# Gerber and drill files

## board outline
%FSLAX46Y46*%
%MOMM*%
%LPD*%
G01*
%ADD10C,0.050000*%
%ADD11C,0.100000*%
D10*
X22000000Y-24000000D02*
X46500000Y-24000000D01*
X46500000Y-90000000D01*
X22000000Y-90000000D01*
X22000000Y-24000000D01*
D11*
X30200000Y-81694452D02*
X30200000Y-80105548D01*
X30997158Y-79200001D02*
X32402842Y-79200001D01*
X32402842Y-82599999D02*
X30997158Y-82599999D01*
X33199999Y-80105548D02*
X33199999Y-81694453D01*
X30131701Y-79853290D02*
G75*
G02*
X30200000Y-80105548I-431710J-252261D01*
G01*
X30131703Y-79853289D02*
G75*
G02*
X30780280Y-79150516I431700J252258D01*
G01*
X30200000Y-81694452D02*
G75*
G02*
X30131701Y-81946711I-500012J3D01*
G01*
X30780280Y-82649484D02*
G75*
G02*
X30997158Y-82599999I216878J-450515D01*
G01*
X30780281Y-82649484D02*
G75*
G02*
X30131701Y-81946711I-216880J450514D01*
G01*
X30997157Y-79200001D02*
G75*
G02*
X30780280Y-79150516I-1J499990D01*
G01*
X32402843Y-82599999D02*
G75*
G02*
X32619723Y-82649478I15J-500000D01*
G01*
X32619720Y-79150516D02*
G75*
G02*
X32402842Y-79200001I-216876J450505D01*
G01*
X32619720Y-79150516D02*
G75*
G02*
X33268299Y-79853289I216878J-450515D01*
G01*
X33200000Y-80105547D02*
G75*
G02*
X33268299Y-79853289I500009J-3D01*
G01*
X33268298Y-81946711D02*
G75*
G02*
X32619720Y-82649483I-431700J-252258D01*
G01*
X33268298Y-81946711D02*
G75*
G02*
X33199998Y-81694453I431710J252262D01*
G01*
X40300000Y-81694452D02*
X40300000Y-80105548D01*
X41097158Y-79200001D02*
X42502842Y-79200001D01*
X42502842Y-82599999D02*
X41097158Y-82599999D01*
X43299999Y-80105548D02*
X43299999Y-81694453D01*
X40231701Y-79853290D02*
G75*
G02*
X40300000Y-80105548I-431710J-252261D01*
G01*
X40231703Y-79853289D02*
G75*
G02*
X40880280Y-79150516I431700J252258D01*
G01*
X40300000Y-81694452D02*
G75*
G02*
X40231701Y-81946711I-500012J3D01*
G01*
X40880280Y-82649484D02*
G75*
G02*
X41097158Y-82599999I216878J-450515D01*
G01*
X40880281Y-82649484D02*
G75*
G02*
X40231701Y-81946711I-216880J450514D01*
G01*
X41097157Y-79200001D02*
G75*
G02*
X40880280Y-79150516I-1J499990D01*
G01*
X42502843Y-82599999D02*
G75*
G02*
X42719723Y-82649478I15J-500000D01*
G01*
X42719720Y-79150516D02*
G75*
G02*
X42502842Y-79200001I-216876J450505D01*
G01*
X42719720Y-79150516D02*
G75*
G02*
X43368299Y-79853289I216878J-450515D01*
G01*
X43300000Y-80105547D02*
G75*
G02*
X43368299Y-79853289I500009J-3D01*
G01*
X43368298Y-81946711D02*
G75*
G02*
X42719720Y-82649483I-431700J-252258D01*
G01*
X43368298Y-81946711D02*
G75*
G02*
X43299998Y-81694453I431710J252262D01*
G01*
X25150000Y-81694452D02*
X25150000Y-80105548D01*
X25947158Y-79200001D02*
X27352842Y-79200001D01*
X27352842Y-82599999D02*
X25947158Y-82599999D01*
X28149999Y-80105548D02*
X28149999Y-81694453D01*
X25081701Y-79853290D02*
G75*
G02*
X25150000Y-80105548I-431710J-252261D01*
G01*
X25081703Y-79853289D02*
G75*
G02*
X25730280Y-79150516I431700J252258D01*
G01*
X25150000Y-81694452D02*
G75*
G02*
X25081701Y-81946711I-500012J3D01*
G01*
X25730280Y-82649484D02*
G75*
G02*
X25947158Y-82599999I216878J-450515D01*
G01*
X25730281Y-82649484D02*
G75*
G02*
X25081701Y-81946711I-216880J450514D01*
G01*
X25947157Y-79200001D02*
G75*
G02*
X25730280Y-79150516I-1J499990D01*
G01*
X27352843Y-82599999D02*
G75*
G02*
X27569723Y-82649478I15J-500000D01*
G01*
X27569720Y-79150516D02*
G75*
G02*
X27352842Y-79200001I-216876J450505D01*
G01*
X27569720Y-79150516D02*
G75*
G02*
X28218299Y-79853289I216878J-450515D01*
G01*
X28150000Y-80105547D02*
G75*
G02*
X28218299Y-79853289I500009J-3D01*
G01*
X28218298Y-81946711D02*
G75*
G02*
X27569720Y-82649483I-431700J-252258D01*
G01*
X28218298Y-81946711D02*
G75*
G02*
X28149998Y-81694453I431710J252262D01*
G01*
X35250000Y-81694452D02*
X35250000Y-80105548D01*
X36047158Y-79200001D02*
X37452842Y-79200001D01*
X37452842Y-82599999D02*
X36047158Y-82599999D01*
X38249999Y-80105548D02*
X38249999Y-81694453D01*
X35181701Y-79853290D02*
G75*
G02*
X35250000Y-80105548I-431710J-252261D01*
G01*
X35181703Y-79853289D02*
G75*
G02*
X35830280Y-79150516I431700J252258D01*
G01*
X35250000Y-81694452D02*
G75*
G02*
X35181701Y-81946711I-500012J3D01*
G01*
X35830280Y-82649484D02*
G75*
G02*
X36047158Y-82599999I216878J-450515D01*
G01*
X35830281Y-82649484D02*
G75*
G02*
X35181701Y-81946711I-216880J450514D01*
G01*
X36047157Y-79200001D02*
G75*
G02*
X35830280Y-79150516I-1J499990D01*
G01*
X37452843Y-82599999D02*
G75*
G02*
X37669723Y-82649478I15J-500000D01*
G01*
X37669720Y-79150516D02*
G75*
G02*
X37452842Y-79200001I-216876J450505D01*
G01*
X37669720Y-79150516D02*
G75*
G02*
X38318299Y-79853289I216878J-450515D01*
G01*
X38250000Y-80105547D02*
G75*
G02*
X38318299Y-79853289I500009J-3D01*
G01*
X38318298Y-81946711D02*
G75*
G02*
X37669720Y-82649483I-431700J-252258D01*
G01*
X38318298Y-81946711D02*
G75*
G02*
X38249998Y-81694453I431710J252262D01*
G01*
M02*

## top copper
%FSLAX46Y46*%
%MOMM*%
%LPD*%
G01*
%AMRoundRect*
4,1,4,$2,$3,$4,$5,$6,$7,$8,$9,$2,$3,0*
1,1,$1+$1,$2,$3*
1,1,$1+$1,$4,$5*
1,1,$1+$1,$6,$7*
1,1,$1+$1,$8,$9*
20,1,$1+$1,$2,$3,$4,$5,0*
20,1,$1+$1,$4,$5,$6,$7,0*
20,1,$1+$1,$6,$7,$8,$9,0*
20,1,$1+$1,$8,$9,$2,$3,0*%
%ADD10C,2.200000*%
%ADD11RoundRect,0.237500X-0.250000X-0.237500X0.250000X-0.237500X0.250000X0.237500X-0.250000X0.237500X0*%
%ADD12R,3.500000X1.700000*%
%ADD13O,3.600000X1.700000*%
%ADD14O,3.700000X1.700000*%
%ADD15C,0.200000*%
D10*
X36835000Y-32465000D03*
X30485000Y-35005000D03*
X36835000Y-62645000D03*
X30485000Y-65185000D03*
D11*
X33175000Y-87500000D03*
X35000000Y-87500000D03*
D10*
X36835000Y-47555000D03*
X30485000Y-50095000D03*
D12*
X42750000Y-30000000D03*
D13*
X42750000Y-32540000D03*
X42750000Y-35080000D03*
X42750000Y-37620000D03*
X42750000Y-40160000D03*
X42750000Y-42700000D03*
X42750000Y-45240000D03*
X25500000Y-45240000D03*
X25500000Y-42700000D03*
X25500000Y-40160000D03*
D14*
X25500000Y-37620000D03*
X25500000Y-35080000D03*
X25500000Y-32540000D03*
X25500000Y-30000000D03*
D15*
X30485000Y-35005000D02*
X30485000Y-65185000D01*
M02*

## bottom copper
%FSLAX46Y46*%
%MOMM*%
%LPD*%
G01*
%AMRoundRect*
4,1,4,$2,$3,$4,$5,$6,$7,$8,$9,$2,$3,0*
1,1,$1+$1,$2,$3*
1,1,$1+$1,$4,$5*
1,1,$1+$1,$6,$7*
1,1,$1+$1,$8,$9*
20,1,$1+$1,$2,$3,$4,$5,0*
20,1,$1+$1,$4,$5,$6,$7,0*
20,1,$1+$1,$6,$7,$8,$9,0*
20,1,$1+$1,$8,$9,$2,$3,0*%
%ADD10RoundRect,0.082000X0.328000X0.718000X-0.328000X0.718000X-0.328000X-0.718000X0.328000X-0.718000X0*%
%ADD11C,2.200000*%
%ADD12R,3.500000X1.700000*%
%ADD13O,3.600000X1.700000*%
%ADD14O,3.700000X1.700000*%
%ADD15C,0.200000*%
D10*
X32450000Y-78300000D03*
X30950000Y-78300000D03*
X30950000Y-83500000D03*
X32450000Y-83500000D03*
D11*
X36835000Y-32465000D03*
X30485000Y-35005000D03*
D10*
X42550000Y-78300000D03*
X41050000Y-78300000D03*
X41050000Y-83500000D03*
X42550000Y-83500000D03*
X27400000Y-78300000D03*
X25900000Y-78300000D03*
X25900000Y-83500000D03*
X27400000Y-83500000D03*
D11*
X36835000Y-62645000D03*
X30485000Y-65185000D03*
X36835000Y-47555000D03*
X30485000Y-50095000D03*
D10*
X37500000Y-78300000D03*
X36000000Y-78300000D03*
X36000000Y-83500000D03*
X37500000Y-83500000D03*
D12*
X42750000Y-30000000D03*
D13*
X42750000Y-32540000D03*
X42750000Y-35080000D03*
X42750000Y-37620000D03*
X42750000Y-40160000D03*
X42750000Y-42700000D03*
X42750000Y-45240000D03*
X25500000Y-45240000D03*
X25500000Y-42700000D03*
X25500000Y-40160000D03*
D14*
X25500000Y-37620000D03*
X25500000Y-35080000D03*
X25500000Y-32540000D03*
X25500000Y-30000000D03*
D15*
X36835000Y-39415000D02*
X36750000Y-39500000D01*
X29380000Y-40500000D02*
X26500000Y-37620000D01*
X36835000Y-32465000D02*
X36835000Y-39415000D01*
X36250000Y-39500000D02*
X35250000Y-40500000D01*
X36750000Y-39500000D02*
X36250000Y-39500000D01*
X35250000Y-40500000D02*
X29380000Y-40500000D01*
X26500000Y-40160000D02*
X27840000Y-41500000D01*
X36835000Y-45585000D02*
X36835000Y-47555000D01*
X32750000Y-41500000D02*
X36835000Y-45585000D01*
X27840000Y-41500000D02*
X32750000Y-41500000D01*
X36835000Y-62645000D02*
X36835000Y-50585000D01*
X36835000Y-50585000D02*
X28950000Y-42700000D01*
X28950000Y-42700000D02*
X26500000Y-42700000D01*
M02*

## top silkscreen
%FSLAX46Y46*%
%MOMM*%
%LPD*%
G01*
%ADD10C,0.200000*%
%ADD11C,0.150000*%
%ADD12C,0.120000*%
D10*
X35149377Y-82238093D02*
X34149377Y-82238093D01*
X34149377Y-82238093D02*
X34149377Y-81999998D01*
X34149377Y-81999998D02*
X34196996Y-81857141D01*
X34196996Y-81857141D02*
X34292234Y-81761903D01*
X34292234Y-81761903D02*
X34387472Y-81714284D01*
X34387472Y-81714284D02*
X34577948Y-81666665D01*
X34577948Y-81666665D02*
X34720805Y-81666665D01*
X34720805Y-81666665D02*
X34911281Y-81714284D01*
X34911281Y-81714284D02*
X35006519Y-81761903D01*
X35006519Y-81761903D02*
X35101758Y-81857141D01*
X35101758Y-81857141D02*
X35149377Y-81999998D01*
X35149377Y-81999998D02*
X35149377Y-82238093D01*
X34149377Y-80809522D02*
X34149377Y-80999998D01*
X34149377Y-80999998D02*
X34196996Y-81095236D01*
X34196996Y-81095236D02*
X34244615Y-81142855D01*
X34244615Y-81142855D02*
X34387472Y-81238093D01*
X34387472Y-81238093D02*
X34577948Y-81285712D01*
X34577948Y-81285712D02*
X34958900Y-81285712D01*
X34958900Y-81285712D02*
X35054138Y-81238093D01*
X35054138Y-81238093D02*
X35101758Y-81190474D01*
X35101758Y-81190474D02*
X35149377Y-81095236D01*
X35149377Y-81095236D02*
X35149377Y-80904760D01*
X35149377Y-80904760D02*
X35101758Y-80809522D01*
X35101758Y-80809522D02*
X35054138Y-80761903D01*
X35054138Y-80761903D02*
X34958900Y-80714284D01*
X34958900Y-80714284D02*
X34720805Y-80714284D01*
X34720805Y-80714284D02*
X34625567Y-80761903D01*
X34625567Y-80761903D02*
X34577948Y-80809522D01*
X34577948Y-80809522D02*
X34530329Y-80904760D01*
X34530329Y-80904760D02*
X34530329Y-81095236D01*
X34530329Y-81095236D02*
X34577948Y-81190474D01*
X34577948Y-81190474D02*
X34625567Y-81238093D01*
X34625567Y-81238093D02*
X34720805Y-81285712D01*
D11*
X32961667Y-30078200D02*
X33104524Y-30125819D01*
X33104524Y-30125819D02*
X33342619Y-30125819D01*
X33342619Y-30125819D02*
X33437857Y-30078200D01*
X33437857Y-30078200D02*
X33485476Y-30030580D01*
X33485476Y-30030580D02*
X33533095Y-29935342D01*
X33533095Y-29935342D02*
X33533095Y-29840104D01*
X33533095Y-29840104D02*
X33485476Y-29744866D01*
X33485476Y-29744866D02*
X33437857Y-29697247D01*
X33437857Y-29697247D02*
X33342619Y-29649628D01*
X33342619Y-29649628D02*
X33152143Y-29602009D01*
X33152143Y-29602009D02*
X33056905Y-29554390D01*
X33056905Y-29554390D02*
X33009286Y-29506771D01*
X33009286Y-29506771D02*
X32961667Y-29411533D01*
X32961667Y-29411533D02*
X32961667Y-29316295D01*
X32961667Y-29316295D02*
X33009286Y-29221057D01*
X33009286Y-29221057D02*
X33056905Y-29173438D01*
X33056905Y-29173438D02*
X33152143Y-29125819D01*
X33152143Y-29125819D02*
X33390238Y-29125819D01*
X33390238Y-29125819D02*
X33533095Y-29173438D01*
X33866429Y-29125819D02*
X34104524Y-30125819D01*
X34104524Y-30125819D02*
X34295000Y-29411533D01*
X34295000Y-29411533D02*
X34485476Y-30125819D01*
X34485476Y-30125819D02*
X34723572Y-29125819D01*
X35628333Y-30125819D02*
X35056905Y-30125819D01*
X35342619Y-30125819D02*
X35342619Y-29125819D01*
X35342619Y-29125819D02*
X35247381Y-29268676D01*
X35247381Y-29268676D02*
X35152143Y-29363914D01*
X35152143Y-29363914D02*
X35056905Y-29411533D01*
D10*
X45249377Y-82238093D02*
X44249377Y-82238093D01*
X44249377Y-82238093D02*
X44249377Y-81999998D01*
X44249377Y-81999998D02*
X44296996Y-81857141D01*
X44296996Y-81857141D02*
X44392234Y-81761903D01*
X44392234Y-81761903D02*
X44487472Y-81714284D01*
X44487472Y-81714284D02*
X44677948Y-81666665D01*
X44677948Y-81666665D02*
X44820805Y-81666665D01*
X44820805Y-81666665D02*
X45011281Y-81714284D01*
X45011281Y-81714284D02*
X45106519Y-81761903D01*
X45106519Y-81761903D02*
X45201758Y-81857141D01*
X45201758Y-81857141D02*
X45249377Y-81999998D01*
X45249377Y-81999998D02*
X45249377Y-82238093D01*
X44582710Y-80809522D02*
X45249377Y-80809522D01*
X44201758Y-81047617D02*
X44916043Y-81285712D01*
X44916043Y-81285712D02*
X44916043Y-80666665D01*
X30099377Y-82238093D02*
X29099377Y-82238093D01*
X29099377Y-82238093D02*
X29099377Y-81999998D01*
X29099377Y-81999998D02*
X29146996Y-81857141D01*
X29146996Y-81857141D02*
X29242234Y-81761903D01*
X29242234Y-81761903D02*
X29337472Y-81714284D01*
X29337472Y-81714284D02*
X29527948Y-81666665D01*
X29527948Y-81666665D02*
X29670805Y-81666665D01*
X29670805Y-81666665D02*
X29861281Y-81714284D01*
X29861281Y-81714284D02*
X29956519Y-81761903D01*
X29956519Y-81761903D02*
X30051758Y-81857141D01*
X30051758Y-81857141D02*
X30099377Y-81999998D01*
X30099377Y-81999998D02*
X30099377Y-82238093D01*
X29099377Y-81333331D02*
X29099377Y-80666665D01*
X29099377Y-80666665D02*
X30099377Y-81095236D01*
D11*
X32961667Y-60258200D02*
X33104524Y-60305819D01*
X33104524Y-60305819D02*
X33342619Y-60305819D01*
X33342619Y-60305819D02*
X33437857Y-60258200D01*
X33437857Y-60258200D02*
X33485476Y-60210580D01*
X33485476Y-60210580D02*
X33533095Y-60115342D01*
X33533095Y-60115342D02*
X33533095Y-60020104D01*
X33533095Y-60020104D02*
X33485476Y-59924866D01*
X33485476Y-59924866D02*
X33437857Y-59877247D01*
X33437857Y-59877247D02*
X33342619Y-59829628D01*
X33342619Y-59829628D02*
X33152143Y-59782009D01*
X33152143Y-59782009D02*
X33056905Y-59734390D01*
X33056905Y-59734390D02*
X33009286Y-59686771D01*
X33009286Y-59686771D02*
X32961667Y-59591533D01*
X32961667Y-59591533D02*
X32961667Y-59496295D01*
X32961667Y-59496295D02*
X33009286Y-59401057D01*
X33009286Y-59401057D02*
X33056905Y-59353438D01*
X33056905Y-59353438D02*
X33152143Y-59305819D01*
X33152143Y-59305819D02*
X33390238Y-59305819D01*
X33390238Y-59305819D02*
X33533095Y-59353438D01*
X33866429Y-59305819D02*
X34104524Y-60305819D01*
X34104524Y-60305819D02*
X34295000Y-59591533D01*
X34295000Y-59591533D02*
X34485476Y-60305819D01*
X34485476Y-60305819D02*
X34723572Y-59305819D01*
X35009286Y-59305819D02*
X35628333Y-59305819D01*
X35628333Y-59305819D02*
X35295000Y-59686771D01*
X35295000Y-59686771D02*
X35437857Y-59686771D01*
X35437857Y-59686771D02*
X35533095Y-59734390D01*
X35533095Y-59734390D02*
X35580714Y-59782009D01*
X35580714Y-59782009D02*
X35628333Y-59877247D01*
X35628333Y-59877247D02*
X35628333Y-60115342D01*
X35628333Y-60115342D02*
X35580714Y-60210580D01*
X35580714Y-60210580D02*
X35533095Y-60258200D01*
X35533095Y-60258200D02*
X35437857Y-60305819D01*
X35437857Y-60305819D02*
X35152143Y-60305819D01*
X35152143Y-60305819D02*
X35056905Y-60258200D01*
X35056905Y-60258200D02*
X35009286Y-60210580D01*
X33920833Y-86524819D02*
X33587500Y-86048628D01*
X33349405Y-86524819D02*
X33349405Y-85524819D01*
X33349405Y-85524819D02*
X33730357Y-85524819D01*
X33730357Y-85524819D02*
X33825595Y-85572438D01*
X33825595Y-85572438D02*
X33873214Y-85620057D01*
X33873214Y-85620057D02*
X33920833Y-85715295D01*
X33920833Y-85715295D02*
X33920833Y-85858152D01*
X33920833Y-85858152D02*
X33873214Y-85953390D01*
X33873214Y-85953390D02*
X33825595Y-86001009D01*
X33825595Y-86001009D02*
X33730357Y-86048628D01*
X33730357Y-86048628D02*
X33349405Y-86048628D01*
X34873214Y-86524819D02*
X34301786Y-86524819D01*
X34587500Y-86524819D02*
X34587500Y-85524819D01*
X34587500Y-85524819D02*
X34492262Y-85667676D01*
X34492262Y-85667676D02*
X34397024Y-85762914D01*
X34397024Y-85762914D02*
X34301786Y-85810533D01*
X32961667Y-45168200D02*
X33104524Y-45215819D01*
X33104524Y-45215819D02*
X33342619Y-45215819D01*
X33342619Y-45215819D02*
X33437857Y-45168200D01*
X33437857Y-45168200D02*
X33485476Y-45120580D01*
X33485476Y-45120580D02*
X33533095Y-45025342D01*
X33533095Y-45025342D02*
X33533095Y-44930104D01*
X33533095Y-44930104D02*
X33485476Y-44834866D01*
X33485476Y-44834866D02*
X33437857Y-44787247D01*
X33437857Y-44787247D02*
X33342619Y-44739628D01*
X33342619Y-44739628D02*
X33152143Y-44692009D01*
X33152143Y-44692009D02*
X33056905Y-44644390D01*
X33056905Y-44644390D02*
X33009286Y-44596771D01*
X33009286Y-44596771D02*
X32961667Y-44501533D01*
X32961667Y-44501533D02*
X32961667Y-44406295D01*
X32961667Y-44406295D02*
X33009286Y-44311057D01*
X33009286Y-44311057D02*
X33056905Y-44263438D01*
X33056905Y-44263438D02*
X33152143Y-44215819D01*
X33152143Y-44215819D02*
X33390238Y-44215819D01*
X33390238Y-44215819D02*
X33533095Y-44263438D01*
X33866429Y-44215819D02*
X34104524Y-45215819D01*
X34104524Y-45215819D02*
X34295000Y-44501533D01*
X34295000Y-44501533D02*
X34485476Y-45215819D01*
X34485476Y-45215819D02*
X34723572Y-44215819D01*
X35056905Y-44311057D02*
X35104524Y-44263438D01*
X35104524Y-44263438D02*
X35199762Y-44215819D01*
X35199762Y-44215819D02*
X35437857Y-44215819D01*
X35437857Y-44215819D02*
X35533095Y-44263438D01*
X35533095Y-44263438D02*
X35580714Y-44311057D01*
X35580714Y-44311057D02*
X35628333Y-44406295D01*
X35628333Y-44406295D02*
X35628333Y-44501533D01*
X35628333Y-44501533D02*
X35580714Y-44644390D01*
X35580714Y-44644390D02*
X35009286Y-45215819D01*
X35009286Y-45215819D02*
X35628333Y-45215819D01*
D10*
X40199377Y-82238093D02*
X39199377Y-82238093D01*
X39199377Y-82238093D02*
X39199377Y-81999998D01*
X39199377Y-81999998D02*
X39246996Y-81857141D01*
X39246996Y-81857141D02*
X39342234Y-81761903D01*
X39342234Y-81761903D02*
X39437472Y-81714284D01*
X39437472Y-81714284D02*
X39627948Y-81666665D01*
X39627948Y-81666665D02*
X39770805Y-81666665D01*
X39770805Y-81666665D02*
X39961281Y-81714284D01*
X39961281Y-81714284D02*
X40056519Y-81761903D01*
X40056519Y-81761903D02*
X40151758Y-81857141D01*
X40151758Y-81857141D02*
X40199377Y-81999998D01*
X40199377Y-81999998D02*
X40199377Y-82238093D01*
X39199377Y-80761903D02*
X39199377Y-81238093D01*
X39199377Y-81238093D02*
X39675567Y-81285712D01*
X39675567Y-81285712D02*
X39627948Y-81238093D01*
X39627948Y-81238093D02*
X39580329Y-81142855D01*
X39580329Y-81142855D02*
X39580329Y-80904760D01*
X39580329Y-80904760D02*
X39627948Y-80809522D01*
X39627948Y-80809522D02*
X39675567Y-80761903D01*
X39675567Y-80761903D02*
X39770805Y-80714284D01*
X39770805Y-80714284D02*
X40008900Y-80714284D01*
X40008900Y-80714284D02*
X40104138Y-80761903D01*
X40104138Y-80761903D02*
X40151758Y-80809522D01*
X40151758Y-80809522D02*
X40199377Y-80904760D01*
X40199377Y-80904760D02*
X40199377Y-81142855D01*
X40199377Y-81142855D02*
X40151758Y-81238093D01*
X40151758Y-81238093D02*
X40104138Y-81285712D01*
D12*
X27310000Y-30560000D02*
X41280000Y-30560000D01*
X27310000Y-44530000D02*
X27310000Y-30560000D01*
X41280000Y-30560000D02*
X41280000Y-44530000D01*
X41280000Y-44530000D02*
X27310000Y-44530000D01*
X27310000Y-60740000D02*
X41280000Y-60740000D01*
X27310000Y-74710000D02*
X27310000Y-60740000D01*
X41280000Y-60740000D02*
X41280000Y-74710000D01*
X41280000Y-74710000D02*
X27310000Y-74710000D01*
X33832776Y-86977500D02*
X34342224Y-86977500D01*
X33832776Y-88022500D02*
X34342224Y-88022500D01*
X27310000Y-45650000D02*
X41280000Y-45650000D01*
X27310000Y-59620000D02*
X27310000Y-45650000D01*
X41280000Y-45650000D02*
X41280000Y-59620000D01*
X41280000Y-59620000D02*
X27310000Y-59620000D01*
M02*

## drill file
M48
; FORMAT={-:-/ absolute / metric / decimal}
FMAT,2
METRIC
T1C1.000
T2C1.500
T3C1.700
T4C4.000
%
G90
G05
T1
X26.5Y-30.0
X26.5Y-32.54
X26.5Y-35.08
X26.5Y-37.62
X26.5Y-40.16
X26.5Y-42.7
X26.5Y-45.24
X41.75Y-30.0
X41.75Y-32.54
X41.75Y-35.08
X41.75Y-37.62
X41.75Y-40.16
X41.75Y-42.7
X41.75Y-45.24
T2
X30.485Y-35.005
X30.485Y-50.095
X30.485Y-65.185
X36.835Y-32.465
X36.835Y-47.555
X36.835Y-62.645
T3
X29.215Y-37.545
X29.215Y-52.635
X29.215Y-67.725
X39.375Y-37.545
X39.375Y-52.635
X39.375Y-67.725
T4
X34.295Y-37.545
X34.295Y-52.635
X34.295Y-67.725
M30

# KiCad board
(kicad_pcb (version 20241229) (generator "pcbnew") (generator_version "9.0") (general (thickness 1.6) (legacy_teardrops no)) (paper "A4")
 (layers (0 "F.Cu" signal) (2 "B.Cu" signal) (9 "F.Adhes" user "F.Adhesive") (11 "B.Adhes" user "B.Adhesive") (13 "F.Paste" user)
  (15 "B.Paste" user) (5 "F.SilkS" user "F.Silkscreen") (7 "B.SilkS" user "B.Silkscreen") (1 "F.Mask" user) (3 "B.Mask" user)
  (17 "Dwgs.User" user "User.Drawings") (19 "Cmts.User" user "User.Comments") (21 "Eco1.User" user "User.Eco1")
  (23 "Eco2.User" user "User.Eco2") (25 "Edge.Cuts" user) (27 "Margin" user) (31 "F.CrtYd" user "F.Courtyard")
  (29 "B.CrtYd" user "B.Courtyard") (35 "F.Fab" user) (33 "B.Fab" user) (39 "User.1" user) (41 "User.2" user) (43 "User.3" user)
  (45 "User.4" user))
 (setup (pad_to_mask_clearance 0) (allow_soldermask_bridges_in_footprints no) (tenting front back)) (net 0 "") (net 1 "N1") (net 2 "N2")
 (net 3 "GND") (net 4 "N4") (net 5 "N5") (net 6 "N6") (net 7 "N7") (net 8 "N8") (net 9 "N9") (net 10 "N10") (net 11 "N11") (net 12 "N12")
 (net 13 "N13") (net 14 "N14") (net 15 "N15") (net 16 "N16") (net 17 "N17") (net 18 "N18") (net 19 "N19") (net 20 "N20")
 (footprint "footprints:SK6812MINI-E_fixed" (layer "F.Cu") (at 31.597158 80.899999 -90)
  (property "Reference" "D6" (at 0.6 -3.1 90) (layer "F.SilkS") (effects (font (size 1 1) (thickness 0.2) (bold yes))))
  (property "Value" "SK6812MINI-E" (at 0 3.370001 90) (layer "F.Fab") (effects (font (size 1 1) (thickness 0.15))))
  (fp_line (start 0.794453 1.397158) (end -0.794451 1.397158) (stroke (width 0.1) (type solid)) (layer "Edge.Cuts"))
  (fp_line (start -1.699998 0.6) (end -1.699998 -0.805684) (stroke (width 0.1) (type solid)) (layer "Edge.Cuts"))
  (fp_line (start 1.7 -0.805684) (end 1.7 0.6) (stroke (width 0.1) (type solid)) (layer "Edge.Cuts"))
  (fp_line (start -0.794451 -1.602841) (end 0.794454 -1.602841) (stroke (width 0.1) (type solid)) (layer "Edge.Cuts"))
  (fp_arc (start -1.046709 1.465457) (mid -0.925121 1.414535) (end -0.794451 1.397158) (stroke (width 0.1) (type solid)) (layer "Edge.Cuts"))
  (fp_arc (start -1.04671 1.465455) (mid -1.638069 1.401192) (end -1.749483 0.816878) (stroke (width 0.1) (type solid)) (layer "Edge.Cuts"))
  (fp_arc (start 0.794453 1.397158) (mid 0.925124 1.414535) (end 1.046712 1.465457) (stroke (width 0.1) (type solid)) (layer "Edge.Cuts"))
  (fp_arc (start 1.749485 0.816878) (mid 1.712528 0.711226) (end 1.7 0.6) (stroke (width 0.1) (type solid)) (layer "Edge.Cuts"))
  (fp_arc (start 1.749485 0.816877) (mid 1.638073 1.401193) (end 1.046712 1.465457) (stroke (width 0.1) (type solid)) (layer "Edge.Cuts"))
  (fp_arc (start -1.699998 0.600001) (mid -1.712526 0.711226) (end -1.749483 0.816878) (stroke (width 0.1) (type solid)) (layer "Edge.Cuts"))
  (fp_arc (start 1.7 -0.805685) (mid 1.712528 -0.91691) (end 1.749485 -1.022562) (stroke (width 0.1) (type solid)) (layer "Edge.Cuts"))
  (fp_arc (start -1.749483 -1.022562) (mid -1.712526 -0.91691) (end -1.699998 -0.805684) (stroke (width 0.1) (type solid))
   (layer "Edge.Cuts"))
  (fp_arc (start -1.749483 -1.022562) (mid -1.63807 -1.606877) (end -1.04671 -1.671141) (stroke (width 0.1) (type solid))
   (layer "Edge.Cuts"))
  (fp_arc (start -0.794452 -1.602842) (mid -0.925122 -1.620219) (end -1.04671 -1.671141) (stroke (width 0.1) (type solid))
   (layer "Edge.Cuts"))
  (fp_arc (start 1.046712 -1.67114) (mid 1.638072 -1.606876) (end 1.749485 -1.022562) (stroke (width 0.1) (type solid)) (layer "Edge.Cuts"))
  (fp_arc (start 1.046712 -1.67114) (mid 0.925124 -1.620218) (end 0.794454 -1.602841) (stroke (width 0.1) (type solid)) (layer "Edge.Cuts"))
  (pad "1" smd roundrect (at -2.599999 -0.852842 180) (size 0.82 1.6) (layers "B.Cu" "B.Mask" "B.Paste") (roundrect_rratio 0.1) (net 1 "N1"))
  (pad "2" smd roundrect (at -2.599999 0.647158 180) (size 0.82 1.6) (layers "B.Cu" "B.Mask" "B.Paste") (roundrect_rratio 0.1) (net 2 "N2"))
  (pad "3" smd roundrect (at 2.600001 0.647158 180) (size 0.82 1.6) (layers "B.Cu" "B.Mask" "B.Paste") (roundrect_rratio 0.1) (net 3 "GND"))
  (pad "4" smd roundrect (at 2.600001 -0.852842 180) (size 0.82 1.6) (layers "B.Cu" "B.Mask" "B.Paste") (roundrect_rratio 0.1) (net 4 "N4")))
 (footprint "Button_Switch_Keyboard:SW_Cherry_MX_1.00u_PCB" (layer "F.Cu") (at 36.835 32.465)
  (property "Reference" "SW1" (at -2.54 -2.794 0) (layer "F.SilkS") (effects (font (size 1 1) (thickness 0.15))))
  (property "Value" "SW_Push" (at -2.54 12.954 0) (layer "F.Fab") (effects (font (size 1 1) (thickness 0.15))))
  (fp_line (start -9.525 -1.905) (end 4.445 -1.905) (stroke (width 0.12) (type solid)) (layer "F.SilkS"))
  (fp_line (start -9.525 12.065) (end -9.525 -1.905) (stroke (width 0.12) (type solid)) (layer "F.SilkS"))
  (fp_line (start 4.445 -1.905) (end 4.445 12.065) (stroke (width 0.12) (type solid)) (layer "F.SilkS"))
  (fp_line (start 4.445 12.065) (end -9.525 12.065) (stroke (width 0.12) (type solid)) (layer "F.SilkS"))
  (pad "" np_thru_hole circle (at -7.62 5.08) (size 1.7 1.7) (drill 1.7) (layers "*.Cu" "*.Mask"))
  (pad "" np_thru_hole circle (at -2.54 5.08) (size 4 4) (drill 4) (layers "*.Cu" "*.Mask"))
  (pad "" np_thru_hole circle (at 2.54 5.08) (size 1.7 1.7) (drill 1.7) (layers "*.Cu" "*.Mask"))
  (pad "1" thru_hole circle (at 0 0) (size 2.2 2.2) (drill 1.5) (layers "*.Cu" "*.Mask") (remove_unused_layers no) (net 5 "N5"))
  (pad "2" thru_hole circle (at -6.35 2.54) (size 2.2 2.2) (drill 1.5) (layers "*.Cu" "*.Mask") (remove_unused_layers no) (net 3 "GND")))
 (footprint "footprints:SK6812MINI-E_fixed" (layer "F.Cu") (at 41.697158 80.899999 -90)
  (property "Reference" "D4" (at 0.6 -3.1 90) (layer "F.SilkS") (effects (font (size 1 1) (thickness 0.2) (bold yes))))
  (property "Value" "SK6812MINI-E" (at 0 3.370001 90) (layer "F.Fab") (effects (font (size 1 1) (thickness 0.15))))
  (fp_line (start 0.794453 1.397158) (end -0.794451 1.397158) (stroke (width 0.1) (type solid)) (layer "Edge.Cuts"))
  (fp_line (start -1.699998 0.6) (end -1.699998 -0.805684) (stroke (width 0.1) (type solid)) (layer "Edge.Cuts"))
  (fp_line (start 1.7 -0.805684) (end 1.7 0.6) (stroke (width 0.1) (type solid)) (layer "Edge.Cuts"))
  (fp_line (start -0.794451 -1.602841) (end 0.794454 -1.602841) (stroke (width 0.1) (type solid)) (layer "Edge.Cuts"))
  (fp_arc (start -1.046709 1.465457) (mid -0.925121 1.414535) (end -0.794451 1.397158) (stroke (width 0.1) (type solid)) (layer "Edge.Cuts"))
  (fp_arc (start -1.04671 1.465455) (mid -1.638069 1.401192) (end -1.749483 0.816878) (stroke (width 0.1) (type solid)) (layer "Edge.Cuts"))
  (fp_arc (start 0.794453 1.397158) (mid 0.925124 1.414535) (end 1.046712 1.465457) (stroke (width 0.1) (type solid)) (layer "Edge.Cuts"))
  (fp_arc (start 1.749485 0.816878) (mid 1.712528 0.711226) (end 1.7 0.6) (stroke (width 0.1) (type solid)) (layer "Edge.Cuts"))
  (fp_arc (start 1.749485 0.816877) (mid 1.638073 1.401193) (end 1.046712 1.465457) (stroke (width 0.1) (type solid)) (layer "Edge.Cuts"))
  (fp_arc (start -1.699998 0.600001) (mid -1.712526 0.711226) (end -1.749483 0.816878) (stroke (width 0.1) (type solid)) (layer "Edge.Cuts"))
  (fp_arc (start 1.7 -0.805685) (mid 1.712528 -0.91691) (end 1.749485 -1.022562) (stroke (width 0.1) (type solid)) (layer "Edge.Cuts"))
  (fp_arc (start -1.749483 -1.022562) (mid -1.712526 -0.91691) (end -1.699998 -0.805684) (stroke (width 0.1) (type solid))
   (layer "Edge.Cuts"))
  (fp_arc (start -1.749483 -1.022562) (mid -1.63807 -1.606877) (end -1.04671 -1.671141) (stroke (width 0.1) (type solid))
   (layer "Edge.Cuts"))
  (fp_arc (start -0.794452 -1.602842) (mid -0.925122 -1.620219) (end -1.04671 -1.671141) (stroke (width 0.1) (type solid))
   (layer "Edge.Cuts"))
  (fp_arc (start 1.046712 -1.67114) (mid 1.638072 -1.606876) (end 1.749485 -1.022562) (stroke (width 0.1) (type solid)) (layer "Edge.Cuts"))
  (fp_arc (start 1.046712 -1.67114) (mid 0.925124 -1.620218) (end 0.794454 -1.602841) (stroke (width 0.1) (type solid)) (layer "Edge.Cuts"))
  (pad "1" smd roundrect (at -2.599999 -0.852842 180) (size 0.82 1.6) (layers "B.Cu" "B.Mask" "B.Paste") (roundrect_rratio 0.1) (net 1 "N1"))
  (pad "2" smd roundrect (at -2.599999 0.647158 180) (size 0.82 1.6) (layers "B.Cu" "B.Mask" "B.Paste") (roundrect_rratio 0.1) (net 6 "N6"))
  (pad "3" smd roundrect (at 2.600001 0.647158 180) (size 0.82 1.6) (layers "B.Cu" "B.Mask" "B.Paste") (roundrect_rratio 0.1) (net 3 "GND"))
  (pad "4" smd roundrect (at 2.600001 -0.852842 180) (size 0.82 1.6) (layers "B.Cu" "B.Mask" "B.Paste") (roundrect_rratio 0.1) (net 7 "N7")))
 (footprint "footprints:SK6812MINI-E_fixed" (layer "F.Cu") (at 26.547158 80.899999 -90)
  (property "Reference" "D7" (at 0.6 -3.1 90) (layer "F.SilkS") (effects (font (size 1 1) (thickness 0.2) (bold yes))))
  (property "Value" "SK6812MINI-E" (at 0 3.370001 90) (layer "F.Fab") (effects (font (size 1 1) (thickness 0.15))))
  (fp_line (start 0.794453 1.397158) (end -0.794451 1.397158) (stroke (width 0.1) (type solid)) (layer "Edge.Cuts"))
  (fp_line (start -1.699998 0.6) (end -1.699998 -0.805684) (stroke (width 0.1) (type solid)) (layer "Edge.Cuts"))
  (fp_line (start 1.7 -0.805684) (end 1.7 0.6) (stroke (width 0.1) (type solid)) (layer "Edge.Cuts"))
  (fp_line (start -0.794451 -1.602841) (end 0.794454 -1.602841) (stroke (width 0.1) (type solid)) (layer "Edge.Cuts"))
  (fp_arc (start -1.046709 1.465457) (mid -0.925121 1.414535) (end -0.794451 1.397158) (stroke (width 0.1) (type solid)) (layer "Edge.Cuts"))
  (fp_arc (start -1.04671 1.465455) (mid -1.638069 1.401192) (end -1.749483 0.816878) (stroke (width 0.1) (type solid)) (layer "Edge.Cuts"))
  (fp_arc (start 0.794453 1.397158) (mid 0.925124 1.414535) (end 1.046712 1.465457) (stroke (width 0.1) (type solid)) (layer "Edge.Cuts"))
  (fp_arc (start 1.749485 0.816878) (mid 1.712528 0.711226) (end 1.7 0.6) (stroke (width 0.1) (type solid)) (layer "Edge.Cuts"))
  (fp_arc (start 1.749485 0.816877) (mid 1.638073 1.401193) (end 1.046712 1.465457) (stroke (width 0.1) (type solid)) (layer "Edge.Cuts"))
  (fp_arc (start -1.699998 0.600001) (mid -1.712526 0.711226) (end -1.749483 0.816878) (stroke (width 0.1) (type solid)) (layer "Edge.Cuts"))
  (fp_arc (start 1.7 -0.805685) (mid 1.712528 -0.91691) (end 1.749485 -1.022562) (stroke (width 0.1) (type solid)) (layer "Edge.Cuts"))
  (fp_arc (start -1.749483 -1.022562) (mid -1.712526 -0.91691) (end -1.699998 -0.805684) (stroke (width 0.1) (type solid))
   (layer "Edge.Cuts"))
  (fp_arc (start -1.749483 -1.022562) (mid -1.63807 -1.606877) (end -1.04671 -1.671141) (stroke (width 0.1) (type solid))
   (layer "Edge.Cuts"))
  (fp_arc (start -0.794452 -1.602842) (mid -0.925122 -1.620219) (end -1.04671 -1.671141) (stroke (width 0.1) (type solid))
   (layer "Edge.Cuts"))
  (fp_arc (start 1.046712 -1.67114) (mid 1.638072 -1.606876) (end 1.749485 -1.022562) (stroke (width 0.1) (type solid)) (layer "Edge.Cuts"))
  (fp_arc (start 1.046712 -1.67114) (mid 0.925124 -1.620218) (end 0.794454 -1.602841) (stroke (width 0.1) (type solid)) (layer "Edge.Cuts"))
  (pad "1" smd roundrect (at -2.599999 -0.852842 180) (size 0.82 1.6) (layers "B.Cu" "B.Mask" "B.Paste") (roundrect_rratio 0.1) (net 1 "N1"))
  (pad "2" smd roundrect (at -2.599999 0.647158 180) (size 0.82 1.6) (layers "B.Cu" "B.Mask" "B.Paste") (roundrect_rratio 0.1) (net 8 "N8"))
  (pad "3" smd roundrect (at 2.600001 0.647158 180) (size 0.82 1.6) (layers "B.Cu" "B.Mask" "B.Paste") (roundrect_rratio 0.1) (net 3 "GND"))
  (pad "4" smd roundrect (at 2.600001 -0.852842 180) (size 0.82 1.6) (layers "B.Cu" "B.Mask" "B.Paste") (roundrect_rratio 0.1) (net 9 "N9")))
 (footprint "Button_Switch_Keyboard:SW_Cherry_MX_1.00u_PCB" (layer "F.Cu") (at 36.835 62.645)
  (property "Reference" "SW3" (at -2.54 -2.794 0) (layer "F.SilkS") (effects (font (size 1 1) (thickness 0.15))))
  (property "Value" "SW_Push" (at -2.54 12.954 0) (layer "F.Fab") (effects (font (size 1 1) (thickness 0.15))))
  (fp_line (start -9.525 -1.905) (end 4.445 -1.905) (stroke (width 0.12) (type solid)) (layer "F.SilkS"))
  (fp_line (start -9.525 12.065) (end -9.525 -1.905) (stroke (width 0.12) (type solid)) (layer "F.SilkS"))
  (fp_line (start 4.445 -1.905) (end 4.445 12.065) (stroke (width 0.12) (type solid)) (layer "F.SilkS"))
  (fp_line (start 4.445 12.065) (end -9.525 12.065) (stroke (width 0.12) (type solid)) (layer "F.SilkS"))
  (pad "" np_thru_hole circle (at -7.62 5.08) (size 1.7 1.7) (drill 1.7) (layers "*.Cu" "*.Mask"))
  (pad "" np_thru_hole circle (at -2.54 5.08) (size 4 4) (drill 4) (layers "*.Cu" "*.Mask"))
  (pad "" np_thru_hole circle (at 2.54 5.08) (size 1.7 1.7) (drill 1.7) (layers "*.Cu" "*.Mask"))
  (pad "1" thru_hole circle (at 0 0) (size 2.2 2.2) (drill 1.5) (layers "*.Cu" "*.Mask") (remove_unused_layers no) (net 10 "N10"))
  (pad "2" thru_hole circle (at -6.35 2.54) (size 2.2 2.2) (drill 1.5) (layers "*.Cu" "*.Mask") (remove_unused_layers no) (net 3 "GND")))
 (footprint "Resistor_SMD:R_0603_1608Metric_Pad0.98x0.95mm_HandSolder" (layer "F.Cu") (at 34.0875 87.5)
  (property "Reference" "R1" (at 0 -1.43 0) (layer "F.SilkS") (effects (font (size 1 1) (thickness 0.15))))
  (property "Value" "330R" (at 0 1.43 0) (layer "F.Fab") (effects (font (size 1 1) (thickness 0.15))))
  (fp_line (start -0.254724 -0.5225) (end 0.254724 -0.5225) (stroke (width 0.12) (type solid)) (layer "F.SilkS"))
  (fp_line (start -0.254724 0.5225) (end 0.254724 0.5225) (stroke (width 0.12) (type solid)) (layer "F.SilkS"))
  (pad "1" smd roundrect (at -0.9125 0) (size 0.975 0.95) (layers "F.Cu" "F.Mask" "F.Paste") (roundrect_rratio 0.25) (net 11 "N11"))
  (pad "2" smd roundrect (at 0.9125 0) (size 0.975 0.95) (layers "F.Cu" "F.Mask" "F.Paste") (roundrect_rratio 0.25) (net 7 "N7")))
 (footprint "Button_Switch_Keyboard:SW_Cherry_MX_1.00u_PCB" (layer "F.Cu") (at 36.835 47.555)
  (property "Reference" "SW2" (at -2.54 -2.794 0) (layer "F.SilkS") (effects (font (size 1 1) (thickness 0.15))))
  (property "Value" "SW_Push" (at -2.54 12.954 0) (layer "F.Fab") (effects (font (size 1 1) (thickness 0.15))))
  (fp_line (start -9.525 -1.905) (end 4.445 -1.905) (stroke (width 0.12) (type solid)) (layer "F.SilkS"))
  (fp_line (start -9.525 12.065) (end -9.525 -1.905) (stroke (width 0.12) (type solid)) (layer "F.SilkS"))
  (fp_line (start 4.445 -1.905) (end 4.445 12.065) (stroke (width 0.12) (type solid)) (layer "F.SilkS"))
  (fp_line (start 4.445 12.065) (end -9.525 12.065) (stroke (width 0.12) (type solid)) (layer "F.SilkS"))
  (pad "" np_thru_hole circle (at -7.62 5.08) (size 1.7 1.7) (drill 1.7) (layers "*.Cu" "*.Mask"))
  (pad "" np_thru_hole circle (at -2.54 5.08) (size 4 4) (drill 4) (layers "*.Cu" "*.Mask"))
  (pad "" np_thru_hole circle (at 2.54 5.08) (size 1.7 1.7) (drill 1.7) (layers "*.Cu" "*.Mask"))
  (pad "1" thru_hole circle (at 0 0) (size 2.2 2.2) (drill 1.5) (layers "*.Cu" "*.Mask") (remove_unused_layers no) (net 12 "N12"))
  (pad "2" thru_hole circle (at -6.35 2.54) (size 2.2 2.2) (drill 1.5) (layers "*.Cu" "*.Mask") (remove_unused_layers no) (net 3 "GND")))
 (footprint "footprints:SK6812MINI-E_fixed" (layer "F.Cu") (at 36.647158 80.899999 -90)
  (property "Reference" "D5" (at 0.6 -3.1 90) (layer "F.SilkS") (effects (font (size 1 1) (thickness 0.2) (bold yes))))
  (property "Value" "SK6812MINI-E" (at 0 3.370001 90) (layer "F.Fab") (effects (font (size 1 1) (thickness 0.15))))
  (fp_line (start 0.794453 1.397158) (end -0.794451 1.397158) (stroke (width 0.1) (type solid)) (layer "Edge.Cuts"))
  (fp_line (start -1.699998 0.6) (end -1.699998 -0.805684) (stroke (width 0.1) (type solid)) (layer "Edge.Cuts"))
  (fp_line (start 1.7 -0.805684) (end 1.7 0.6) (stroke (width 0.1) (type solid)) (layer "Edge.Cuts"))
  (fp_line (start -0.794451 -1.602841) (end 0.794454 -1.602841) (stroke (width 0.1) (type solid)) (layer "Edge.Cuts"))
  (fp_arc (start -1.046709 1.465457) (mid -0.925121 1.414535) (end -0.794451 1.397158) (stroke (width 0.1) (type solid)) (layer "Edge.Cuts"))
  (fp_arc (start -1.04671 1.465455) (mid -1.638069 1.401192) (end -1.749483 0.816878) (stroke (width 0.1) (type solid)) (layer "Edge.Cuts"))
  (fp_arc (start 0.794453 1.397158) (mid 0.925124 1.414535) (end 1.046712 1.465457) (stroke (width 0.1) (type solid)) (layer "Edge.Cuts"))
  (fp_arc (start 1.749485 0.816878) (mid 1.712528 0.711226) (end 1.7 0.6) (stroke (width 0.1) (type solid)) (layer "Edge.Cuts"))
  (fp_arc (start 1.749485 0.816877) (mid 1.638073 1.401193) (end 1.046712 1.465457) (stroke (width 0.1) (type solid)) (layer "Edge.Cuts"))
  (fp_arc (start -1.699998 0.600001) (mid -1.712526 0.711226) (end -1.749483 0.816878) (stroke (width 0.1) (type solid)) (layer "Edge.Cuts"))
  (fp_arc (start 1.7 -0.805685) (mid 1.712528 -0.91691) (end 1.749485 -1.022562) (stroke (width 0.1) (type solid)) (layer "Edge.Cuts"))
  (fp_arc (start -1.749483 -1.022562) (mid -1.712526 -0.91691) (end -1.699998 -0.805684) (stroke (width 0.1) (type solid))
   (layer "Edge.Cuts"))
  (fp_arc (start -1.749483 -1.022562) (mid -1.63807 -1.606877) (end -1.04671 -1.671141) (stroke (width 0.1) (type solid))
   (layer "Edge.Cuts"))
  (fp_arc (start -0.794452 -1.602842) (mid -0.925122 -1.620219) (end -1.04671 -1.671141) (stroke (width 0.1) (type solid))
   (layer "Edge.Cuts"))
  (fp_arc (start 1.046712 -1.67114) (mid 1.638072 -1.606876) (end 1.749485 -1.022562) (stroke (width 0.1) (type solid)) (layer "Edge.Cuts"))
  (fp_arc (start 1.046712 -1.67114) (mid 0.925124 -1.620218) (end 0.794454 -1.602841) (stroke (width 0.1) (type solid)) (layer "Edge.Cuts"))
  (pad "1" smd roundrect (at -2.599999 -0.852842 180) (size 0.82 1.6) (layers "B.Cu" "B.Mask" "B.Paste") (roundrect_rratio 0.1) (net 1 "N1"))
  (pad "2" smd roundrect (at -2.599999 0.647158 180) (size 0.82 1.6) (layers "B.Cu" "B.Mask" "B.Paste") (roundrect_rratio 0.1) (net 4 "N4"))
  (pad "3" smd roundrect (at 2.600001 0.647158 180) (size 0.82 1.6) (layers "B.Cu" "B.Mask" "B.Paste") (roundrect_rratio 0.1) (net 3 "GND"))
  (pad "4" smd roundrect (at 2.600001 -0.852842 180) (size 0.82 1.6) (layers "B.Cu" "B.Mask" "B.Paste") (roundrect_rratio 0.1) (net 6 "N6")))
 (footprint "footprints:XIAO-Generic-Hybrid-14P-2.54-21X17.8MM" (layer "B.Cu") (at 34.125 37.62 180)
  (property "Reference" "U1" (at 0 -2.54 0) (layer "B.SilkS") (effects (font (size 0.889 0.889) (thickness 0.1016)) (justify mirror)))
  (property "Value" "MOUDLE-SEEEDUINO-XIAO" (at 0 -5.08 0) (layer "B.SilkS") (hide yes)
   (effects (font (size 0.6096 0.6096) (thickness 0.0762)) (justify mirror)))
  (pad "1" thru_hole rect (at -7.625 7.62 180) (size 3.5 1.7) (drill 1 (offset -1 0)) (layers "*.Cu" "*.Mask") (remove_unused_layers no)
   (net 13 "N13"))
  (pad "2" thru_hole oval (at -7.625 5.08 180) (size 3.6 1.7) (drill 1 (offset -1 0)) (layers "*.Cu" "*.Mask") (remove_unused_layers no)
   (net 11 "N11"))
  (pad "3" thru_hole oval (at -7.625 2.54 180) (size 3.6 1.7) (drill 1 (offset -1 0)) (layers "*.Cu" "*.Mask") (remove_unused_layers no)
   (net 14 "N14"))
  (pad "4" thru_hole oval (at -7.625 0 180) (size 3.6 1.7) (drill 1 (offset -1 0)) (layers "*.Cu" "*.Mask") (remove_unused_layers no)
   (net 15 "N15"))
  (pad "5" thru_hole oval (at -7.625 -2.54 180) (size 3.6 1.7) (drill 1 (offset -1 0)) (layers "*.Cu" "*.Mask") (remove_unused_layers no)
   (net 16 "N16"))
  (pad "6" thru_hole oval (at -7.625 -5.08) (size 3.6 1.7) (drill 1 (offset 1 0)) (layers "*.Cu" "*.Mask") (remove_unused_layers no)
   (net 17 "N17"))
  (pad "7" thru_hole oval (at -7.625 -7.62 180) (size 3.6 1.7) (drill 1 (offset -1 0)) (layers "*.Cu" "*.Mask") (remove_unused_layers no)
   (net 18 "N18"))
  (pad "8" thru_hole oval (at 7.625 -7.62 180) (size 3.6 1.7) (drill 1 (offset 1 0)) (layers "*.Cu" "*.Mask") (remove_unused_layers no)
   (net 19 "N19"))
  (pad "9" thru_hole oval (at 7.625 -5.08 180) (size 3.6 1.7) (drill 1 (offset 1 0)) (layers "*.Cu" "*.Mask") (remove_unused_layers no)
   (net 10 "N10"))
  (pad "10" thru_hole oval (at 7.625 -2.54 180) (size 3.6 1.7) (drill 1 (offset 1 0)) (layers "*.Cu" "*.Mask") (remove_unused_layers no)
   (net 12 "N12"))
  (pad "11" thru_hole oval (at 7.625 0 180) (size 3.7 1.7) (drill 1 (offset 1 0)) (layers "*.Cu" "*.Mask") (remove_unused_layers no)
   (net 5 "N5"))
  (pad "12" thru_hole oval (at 7.625 2.54 180) (size 3.7 1.7) (drill 1 (offset 1 0)) (layers "*.Cu" "*.Mask") (remove_unused_layers no)
   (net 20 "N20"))
  (pad "13" thru_hole oval (at 7.625 5.08 180) (size 3.7 1.7) (drill 1 (offset 1 0)) (layers "*.Cu" "*.Mask") (remove_unused_layers no)
   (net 3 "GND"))
  (pad "14" thru_hole oval (at 7.625 7.62 180) (size 3.7 1.7) (drill 1 (offset 1 0)) (layers "*.Cu" "*.Mask") (remove_unused_layers no)
   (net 1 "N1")))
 (gr_rect (start 22 24) (end 46.5 90) (stroke (width 0.05) (type default)) (fill no) (layer "Edge.Cuts"))
 (segment (start 36.835 39.415) (end 36.75 39.5) (width 0.2) (layer "B.Cu") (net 5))
 (segment (start 29.38 40.5) (end 26.5 37.62) (width 0.2) (layer "B.Cu") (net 5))
 (segment (start 36.835 32.465) (end 36.835 39.415) (width 0.2) (layer "B.Cu") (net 5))
 (segment (start 36.25 39.5) (end 35.25 40.5) (width 0.2) (layer "B.Cu") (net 5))
 (segment (start 36.75 39.5) (end 36.25 39.5) (width 0.2) (layer "B.Cu") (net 5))
 (segment (start 35.25 40.5) (end 29.38 40.5) (width 0.2) (layer "B.Cu") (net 5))
 (segment (start 30.485 35.005) (end 30.485 65.185) (width 0.2) (layer "F.Cu") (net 3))
 (segment (start 26.5 40.16) (end 27.84 41.5) (width 0.2) (layer "B.Cu") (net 12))
 (segment (start 36.835 45.585) (end 36.835 47.555) (width 0.2) (layer "B.Cu") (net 12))
 (segment (start 32.75 41.5) (end 36.835 45.585) (width 0.2) (layer "B.Cu") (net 12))
 (segment (start 27.84 41.5) (end 32.75 41.5) (width 0.2) (layer "B.Cu") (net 12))
 (segment (start 36.835 62.645) (end 36.835 50.585) (width 0.2) (layer "B.Cu") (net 10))
 (segment (start 36.835 50.585) (end 28.95 42.7) (width 0.2) (layer "B.Cu") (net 10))
 (segment (start 28.95 42.7) (end 26.5 42.7) (width 0.2) (layer "B.Cu") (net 10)))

